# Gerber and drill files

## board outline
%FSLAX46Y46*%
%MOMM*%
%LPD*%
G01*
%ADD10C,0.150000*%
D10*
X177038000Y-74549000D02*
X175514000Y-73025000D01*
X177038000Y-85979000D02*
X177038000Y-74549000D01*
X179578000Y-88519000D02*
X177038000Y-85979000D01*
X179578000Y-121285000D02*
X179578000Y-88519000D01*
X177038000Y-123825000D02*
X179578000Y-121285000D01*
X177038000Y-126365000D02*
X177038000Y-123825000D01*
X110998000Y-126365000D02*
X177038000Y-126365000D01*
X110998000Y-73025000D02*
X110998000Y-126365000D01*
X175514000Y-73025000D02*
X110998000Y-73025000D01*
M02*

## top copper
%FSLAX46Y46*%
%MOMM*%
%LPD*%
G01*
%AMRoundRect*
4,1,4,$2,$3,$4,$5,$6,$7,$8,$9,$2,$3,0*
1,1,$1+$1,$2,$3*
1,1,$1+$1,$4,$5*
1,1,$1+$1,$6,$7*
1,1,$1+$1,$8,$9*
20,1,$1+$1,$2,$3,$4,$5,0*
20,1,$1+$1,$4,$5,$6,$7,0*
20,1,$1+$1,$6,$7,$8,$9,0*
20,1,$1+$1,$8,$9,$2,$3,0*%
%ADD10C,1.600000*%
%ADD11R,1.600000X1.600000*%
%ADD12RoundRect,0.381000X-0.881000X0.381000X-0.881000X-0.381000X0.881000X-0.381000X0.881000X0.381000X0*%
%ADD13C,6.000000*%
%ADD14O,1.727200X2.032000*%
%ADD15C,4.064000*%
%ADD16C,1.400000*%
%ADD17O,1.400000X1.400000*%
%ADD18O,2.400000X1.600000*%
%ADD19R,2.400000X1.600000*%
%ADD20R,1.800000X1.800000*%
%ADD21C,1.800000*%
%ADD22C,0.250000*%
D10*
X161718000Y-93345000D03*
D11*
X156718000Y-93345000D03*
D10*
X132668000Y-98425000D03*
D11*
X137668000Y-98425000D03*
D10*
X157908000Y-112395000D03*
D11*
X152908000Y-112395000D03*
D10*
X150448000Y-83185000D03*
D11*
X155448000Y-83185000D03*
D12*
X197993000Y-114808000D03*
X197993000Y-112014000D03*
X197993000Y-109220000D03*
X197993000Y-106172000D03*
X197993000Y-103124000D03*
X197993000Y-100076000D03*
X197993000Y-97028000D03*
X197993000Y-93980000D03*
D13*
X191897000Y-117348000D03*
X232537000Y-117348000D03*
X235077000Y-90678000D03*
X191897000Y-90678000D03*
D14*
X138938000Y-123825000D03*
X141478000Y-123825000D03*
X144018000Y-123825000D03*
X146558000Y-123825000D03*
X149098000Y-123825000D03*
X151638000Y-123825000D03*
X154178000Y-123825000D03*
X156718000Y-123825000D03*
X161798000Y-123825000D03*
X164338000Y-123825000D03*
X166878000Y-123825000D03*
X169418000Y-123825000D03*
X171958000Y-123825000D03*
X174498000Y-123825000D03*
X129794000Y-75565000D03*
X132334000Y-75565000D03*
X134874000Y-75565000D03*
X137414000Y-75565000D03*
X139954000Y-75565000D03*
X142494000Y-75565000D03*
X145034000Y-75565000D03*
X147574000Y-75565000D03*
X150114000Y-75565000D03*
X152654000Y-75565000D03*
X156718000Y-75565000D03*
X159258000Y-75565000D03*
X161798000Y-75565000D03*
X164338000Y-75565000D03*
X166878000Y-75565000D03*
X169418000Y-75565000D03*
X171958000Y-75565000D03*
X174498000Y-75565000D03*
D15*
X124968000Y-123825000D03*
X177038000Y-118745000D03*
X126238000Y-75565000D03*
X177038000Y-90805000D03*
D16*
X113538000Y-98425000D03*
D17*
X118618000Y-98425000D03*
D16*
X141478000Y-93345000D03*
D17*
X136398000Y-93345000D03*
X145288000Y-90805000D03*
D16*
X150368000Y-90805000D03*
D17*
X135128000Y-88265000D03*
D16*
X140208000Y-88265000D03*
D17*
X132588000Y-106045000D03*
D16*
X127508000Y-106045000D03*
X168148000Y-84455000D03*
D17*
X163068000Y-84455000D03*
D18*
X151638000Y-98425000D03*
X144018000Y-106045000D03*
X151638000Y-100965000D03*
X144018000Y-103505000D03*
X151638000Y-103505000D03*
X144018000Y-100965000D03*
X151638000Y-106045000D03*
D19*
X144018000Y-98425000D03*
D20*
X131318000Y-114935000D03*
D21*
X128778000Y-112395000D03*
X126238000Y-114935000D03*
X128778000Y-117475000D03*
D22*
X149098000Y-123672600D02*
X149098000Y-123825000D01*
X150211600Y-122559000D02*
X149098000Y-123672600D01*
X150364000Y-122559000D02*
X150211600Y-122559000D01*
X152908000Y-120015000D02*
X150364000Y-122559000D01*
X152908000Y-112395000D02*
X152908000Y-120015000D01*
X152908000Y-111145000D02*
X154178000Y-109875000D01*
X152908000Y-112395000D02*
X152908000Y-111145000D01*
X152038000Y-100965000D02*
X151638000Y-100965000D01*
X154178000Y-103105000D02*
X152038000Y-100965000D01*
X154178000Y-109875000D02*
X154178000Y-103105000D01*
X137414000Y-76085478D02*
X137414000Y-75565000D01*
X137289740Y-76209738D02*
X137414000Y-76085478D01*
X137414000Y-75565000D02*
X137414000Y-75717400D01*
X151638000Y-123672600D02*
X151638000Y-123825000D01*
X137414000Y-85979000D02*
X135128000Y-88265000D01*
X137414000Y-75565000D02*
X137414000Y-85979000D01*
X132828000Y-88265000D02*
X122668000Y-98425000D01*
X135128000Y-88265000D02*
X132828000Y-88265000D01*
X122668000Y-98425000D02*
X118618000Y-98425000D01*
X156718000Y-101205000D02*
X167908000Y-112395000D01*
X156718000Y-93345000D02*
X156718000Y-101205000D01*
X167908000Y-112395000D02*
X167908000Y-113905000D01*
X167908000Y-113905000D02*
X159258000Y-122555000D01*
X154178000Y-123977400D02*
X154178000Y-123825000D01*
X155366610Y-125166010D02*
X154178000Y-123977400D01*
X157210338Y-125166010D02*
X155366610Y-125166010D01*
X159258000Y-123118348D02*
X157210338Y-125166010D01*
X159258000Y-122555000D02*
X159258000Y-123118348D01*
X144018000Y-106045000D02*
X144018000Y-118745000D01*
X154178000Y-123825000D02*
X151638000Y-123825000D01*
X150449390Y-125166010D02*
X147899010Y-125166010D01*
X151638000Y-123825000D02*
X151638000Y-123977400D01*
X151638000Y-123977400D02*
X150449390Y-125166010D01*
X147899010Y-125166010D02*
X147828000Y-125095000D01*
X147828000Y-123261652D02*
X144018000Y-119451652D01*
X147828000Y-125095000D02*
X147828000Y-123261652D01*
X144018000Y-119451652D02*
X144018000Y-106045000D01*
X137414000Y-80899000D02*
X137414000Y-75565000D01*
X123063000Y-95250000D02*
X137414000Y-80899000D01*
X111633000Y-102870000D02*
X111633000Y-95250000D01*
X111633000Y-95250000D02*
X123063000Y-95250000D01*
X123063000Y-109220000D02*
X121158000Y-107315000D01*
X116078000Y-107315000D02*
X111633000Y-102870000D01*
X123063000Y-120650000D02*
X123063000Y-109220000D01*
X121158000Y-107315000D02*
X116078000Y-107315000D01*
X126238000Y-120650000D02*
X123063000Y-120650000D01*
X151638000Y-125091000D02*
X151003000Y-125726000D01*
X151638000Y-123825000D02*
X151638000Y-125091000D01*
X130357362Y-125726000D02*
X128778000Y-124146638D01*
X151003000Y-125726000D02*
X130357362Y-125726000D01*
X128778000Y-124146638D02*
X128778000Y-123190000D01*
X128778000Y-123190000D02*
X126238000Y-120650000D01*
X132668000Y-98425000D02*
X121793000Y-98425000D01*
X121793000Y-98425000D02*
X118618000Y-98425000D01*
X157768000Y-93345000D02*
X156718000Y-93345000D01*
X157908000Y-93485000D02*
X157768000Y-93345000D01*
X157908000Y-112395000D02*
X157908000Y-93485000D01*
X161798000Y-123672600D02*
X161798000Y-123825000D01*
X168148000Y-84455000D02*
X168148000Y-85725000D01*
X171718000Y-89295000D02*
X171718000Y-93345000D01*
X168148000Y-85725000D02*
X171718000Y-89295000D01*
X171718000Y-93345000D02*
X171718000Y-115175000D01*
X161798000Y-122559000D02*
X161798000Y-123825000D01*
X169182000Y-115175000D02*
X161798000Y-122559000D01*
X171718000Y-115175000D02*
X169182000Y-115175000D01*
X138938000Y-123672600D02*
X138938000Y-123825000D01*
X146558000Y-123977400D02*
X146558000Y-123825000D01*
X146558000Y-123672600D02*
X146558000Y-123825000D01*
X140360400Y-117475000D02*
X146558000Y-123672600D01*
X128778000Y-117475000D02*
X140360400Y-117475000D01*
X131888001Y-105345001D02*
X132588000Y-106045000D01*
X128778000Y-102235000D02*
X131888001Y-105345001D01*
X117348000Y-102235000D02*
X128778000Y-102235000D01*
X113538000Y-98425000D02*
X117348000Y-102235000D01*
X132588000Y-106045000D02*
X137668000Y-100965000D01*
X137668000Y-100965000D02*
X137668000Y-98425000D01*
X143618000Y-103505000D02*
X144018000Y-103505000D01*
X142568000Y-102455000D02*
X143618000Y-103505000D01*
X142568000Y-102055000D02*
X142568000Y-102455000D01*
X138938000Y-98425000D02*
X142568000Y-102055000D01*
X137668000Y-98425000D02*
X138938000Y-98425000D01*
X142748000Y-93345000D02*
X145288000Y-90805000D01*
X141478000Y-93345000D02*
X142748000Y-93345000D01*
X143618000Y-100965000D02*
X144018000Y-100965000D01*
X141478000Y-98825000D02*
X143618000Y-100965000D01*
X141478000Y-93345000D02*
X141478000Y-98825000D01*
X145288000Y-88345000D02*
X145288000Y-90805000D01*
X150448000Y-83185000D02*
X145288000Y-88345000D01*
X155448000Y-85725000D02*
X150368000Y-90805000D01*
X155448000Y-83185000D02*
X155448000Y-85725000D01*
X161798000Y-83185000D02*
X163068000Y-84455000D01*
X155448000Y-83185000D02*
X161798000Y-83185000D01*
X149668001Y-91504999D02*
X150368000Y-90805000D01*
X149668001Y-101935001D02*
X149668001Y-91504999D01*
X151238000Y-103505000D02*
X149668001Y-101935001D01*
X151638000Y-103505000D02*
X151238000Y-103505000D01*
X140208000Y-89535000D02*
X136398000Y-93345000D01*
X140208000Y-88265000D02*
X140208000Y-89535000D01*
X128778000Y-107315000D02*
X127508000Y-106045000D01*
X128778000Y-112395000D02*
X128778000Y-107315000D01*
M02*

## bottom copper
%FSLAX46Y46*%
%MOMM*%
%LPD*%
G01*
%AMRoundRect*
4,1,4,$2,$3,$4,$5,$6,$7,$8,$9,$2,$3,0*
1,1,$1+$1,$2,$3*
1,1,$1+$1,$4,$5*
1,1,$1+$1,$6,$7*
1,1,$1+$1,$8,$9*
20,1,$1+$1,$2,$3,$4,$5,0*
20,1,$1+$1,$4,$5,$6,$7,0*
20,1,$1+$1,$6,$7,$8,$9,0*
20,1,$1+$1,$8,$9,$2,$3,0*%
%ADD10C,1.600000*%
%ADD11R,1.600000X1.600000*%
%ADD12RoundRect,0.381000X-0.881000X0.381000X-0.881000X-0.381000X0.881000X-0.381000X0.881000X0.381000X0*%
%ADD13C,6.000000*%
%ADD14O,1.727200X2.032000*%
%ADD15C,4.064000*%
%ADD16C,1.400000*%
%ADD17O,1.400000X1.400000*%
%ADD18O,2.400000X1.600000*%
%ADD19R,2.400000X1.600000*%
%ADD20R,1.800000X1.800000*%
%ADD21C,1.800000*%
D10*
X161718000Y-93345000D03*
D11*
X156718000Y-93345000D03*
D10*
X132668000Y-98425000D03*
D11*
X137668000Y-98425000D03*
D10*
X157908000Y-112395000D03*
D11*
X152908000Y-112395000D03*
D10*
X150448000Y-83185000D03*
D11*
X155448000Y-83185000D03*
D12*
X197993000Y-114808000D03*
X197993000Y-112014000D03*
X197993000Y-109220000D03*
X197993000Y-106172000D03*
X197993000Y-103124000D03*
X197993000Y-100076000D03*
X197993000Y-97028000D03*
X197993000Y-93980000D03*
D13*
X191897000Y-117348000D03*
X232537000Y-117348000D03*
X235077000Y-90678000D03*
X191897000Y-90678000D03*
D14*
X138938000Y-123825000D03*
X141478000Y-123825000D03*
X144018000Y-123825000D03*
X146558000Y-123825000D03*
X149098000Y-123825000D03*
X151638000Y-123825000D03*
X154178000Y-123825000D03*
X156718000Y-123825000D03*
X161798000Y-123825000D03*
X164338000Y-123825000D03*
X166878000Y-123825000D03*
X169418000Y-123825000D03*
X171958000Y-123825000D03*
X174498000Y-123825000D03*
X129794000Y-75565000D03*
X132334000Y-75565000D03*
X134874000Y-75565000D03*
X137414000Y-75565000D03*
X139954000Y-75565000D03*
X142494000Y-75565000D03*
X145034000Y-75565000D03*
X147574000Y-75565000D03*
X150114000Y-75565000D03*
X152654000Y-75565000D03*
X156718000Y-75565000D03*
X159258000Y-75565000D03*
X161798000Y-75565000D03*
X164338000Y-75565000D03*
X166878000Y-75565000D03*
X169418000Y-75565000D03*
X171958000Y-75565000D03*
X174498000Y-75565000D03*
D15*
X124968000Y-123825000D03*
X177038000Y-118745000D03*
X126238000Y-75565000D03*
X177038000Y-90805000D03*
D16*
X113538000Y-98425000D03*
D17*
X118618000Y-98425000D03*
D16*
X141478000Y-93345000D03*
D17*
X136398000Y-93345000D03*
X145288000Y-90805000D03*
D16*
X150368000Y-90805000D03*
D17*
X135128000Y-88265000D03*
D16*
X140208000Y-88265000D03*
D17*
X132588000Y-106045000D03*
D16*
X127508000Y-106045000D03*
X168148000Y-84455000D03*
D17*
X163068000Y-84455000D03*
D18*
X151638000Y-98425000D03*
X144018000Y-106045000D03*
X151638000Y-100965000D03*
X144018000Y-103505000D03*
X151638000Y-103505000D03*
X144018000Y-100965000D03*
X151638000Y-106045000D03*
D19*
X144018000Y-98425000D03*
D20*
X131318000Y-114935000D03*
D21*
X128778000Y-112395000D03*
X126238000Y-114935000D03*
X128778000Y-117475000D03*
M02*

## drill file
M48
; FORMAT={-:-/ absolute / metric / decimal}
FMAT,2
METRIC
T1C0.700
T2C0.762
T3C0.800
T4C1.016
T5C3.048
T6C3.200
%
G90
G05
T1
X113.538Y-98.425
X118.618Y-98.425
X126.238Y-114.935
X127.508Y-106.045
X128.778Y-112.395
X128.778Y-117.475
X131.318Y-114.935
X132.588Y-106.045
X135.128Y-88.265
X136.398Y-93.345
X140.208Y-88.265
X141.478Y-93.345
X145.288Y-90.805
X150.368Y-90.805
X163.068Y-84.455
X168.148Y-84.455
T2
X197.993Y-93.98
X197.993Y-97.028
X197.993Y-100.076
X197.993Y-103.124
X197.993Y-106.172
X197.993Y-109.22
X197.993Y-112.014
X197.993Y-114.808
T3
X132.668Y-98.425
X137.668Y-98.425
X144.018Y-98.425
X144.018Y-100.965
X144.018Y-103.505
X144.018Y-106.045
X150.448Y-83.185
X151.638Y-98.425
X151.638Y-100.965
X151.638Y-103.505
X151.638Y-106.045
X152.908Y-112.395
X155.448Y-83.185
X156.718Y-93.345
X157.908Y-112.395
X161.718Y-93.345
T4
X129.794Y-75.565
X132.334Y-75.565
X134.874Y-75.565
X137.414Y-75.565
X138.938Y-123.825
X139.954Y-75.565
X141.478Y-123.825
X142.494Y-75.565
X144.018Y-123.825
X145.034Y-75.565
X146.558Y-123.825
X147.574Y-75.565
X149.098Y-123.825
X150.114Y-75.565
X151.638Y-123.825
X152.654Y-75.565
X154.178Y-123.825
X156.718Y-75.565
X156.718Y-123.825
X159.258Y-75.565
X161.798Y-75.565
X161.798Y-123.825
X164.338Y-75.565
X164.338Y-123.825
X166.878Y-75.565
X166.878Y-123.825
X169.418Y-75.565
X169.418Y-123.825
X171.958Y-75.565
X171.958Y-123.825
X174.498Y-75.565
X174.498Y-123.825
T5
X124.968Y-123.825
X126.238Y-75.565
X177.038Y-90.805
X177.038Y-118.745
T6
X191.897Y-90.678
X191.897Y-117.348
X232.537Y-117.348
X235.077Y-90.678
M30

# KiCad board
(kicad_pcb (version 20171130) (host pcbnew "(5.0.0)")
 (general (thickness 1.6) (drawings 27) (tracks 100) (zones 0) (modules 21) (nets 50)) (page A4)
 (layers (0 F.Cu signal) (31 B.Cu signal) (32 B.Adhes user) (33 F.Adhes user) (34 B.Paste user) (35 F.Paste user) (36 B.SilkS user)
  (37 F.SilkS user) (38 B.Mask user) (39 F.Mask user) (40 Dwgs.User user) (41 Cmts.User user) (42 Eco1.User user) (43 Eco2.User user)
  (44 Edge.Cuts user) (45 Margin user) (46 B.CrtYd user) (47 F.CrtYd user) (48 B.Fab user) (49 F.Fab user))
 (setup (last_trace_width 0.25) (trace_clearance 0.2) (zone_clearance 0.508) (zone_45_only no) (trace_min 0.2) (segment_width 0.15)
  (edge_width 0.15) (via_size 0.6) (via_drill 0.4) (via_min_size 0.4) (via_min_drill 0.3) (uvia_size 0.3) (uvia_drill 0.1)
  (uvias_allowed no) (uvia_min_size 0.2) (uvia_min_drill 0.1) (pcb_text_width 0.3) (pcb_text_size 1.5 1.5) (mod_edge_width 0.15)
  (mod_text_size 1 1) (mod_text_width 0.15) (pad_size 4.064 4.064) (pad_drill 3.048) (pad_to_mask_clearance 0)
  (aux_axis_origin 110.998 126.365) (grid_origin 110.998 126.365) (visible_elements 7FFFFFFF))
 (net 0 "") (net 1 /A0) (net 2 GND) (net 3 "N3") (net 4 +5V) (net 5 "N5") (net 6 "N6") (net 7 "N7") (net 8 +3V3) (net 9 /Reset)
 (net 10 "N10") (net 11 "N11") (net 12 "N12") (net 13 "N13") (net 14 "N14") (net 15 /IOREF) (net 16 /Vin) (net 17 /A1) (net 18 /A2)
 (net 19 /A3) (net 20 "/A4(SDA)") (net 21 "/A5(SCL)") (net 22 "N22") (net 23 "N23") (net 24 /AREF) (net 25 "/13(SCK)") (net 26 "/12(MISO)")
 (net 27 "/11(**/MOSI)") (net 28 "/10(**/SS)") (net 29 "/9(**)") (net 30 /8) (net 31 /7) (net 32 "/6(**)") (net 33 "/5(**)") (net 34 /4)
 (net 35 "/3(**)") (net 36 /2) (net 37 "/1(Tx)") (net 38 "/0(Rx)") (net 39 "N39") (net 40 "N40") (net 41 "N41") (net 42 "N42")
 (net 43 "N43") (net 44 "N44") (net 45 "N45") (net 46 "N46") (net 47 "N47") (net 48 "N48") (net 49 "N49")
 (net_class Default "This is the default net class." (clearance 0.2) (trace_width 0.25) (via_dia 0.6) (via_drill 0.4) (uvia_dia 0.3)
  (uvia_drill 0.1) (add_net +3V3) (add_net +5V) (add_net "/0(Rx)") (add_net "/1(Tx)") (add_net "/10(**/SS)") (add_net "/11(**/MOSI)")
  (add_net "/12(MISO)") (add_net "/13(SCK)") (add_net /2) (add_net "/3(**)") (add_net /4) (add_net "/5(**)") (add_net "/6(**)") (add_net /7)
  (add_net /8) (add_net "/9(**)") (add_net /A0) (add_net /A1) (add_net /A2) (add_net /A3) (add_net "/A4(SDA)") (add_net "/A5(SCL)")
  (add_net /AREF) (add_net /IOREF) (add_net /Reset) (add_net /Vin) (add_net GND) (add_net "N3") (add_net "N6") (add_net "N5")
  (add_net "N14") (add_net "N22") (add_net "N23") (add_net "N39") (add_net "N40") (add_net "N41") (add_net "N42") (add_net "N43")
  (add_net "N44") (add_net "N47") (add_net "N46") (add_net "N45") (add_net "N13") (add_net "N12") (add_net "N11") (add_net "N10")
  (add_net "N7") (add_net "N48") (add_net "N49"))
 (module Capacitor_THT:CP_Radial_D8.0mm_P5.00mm (layer F.Cu) (at 156.718 93.345)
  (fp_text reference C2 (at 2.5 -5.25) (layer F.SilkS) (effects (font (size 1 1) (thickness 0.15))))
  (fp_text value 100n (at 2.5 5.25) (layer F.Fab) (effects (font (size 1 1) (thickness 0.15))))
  (pad 2 thru_hole circle (at 5 0) (size 1.6 1.6) (drill 0.8) (layers *.Cu *.Mask) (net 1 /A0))
  (pad 1 thru_hole rect (at 0 0) (size 1.6 1.6) (drill 0.8) (layers *.Cu *.Mask) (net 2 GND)))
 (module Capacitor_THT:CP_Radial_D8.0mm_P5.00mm (layer F.Cu) (at 137.668 98.425 180)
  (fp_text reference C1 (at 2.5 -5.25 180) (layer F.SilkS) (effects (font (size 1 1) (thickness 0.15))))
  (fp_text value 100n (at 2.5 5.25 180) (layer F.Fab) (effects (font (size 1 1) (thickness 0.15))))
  (pad 2 thru_hole circle (at 5 0 180) (size 1.6 1.6) (drill 0.8) (layers *.Cu *.Mask) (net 2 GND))
  (pad 1 thru_hole rect (at 0 0 180) (size 1.6 1.6) (drill 0.8) (layers *.Cu *.Mask) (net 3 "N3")))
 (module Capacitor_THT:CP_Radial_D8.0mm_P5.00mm (layer F.Cu) (at 152.908 112.395)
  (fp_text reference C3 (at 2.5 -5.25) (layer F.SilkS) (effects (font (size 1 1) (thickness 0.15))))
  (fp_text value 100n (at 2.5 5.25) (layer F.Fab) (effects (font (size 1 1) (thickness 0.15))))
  (pad 2 thru_hole circle (at 5 0) (size 1.6 1.6) (drill 0.8) (layers *.Cu *.Mask) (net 2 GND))
  (pad 1 thru_hole rect (at 0 0) (size 1.6 1.6) (drill 0.8) (layers *.Cu *.Mask) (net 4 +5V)))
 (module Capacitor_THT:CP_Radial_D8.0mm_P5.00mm (layer F.Cu) (at 155.448 83.185 180)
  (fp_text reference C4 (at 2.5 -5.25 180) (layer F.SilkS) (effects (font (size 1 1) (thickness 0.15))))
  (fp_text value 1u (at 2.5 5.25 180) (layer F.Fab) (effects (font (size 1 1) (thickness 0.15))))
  (pad 2 thru_hole circle (at 5 0 180) (size 1.6 1.6) (drill 0.8) (layers *.Cu *.Mask) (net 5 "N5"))
  (pad 1 thru_hole rect (at 0 0 180) (size 1.6 1.6) (drill 0.8) (layers *.Cu *.Mask) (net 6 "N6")))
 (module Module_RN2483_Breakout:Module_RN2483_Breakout (layer F.Cu) (at 197.993 93.98 270)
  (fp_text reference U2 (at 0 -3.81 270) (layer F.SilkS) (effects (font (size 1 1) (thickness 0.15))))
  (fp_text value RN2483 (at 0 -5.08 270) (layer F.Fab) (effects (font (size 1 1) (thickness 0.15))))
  (pad 8 thru_hole roundrect (at 20.828 0 270) (size 1.524 2.524) (drill 0.762) (layers *.Cu *.Mask) (roundrect_rratio 0.25) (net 2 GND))
  (pad 7 thru_hole roundrect (at 18.034 0 270) (size 1.524 2.524) (drill 0.762) (layers *.Cu *.Mask) (roundrect_rratio 0.25) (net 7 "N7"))
  (pad 6 thru_hole roundrect (at 15.24 0 270) (size 1.524 2.524) (drill 0.762) (layers *.Cu *.Mask) (roundrect_rratio 0.25) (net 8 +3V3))
  (pad 5 thru_hole roundrect (at 12.192 0 270) (size 1.524 2.524) (drill 0.762) (layers *.Cu *.Mask) (roundrect_rratio 0.25) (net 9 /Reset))
  (pad 4 thru_hole roundrect (at 9.144 0 270) (size 1.524 2.524) (drill 0.762) (layers *.Cu *.Mask) (roundrect_rratio 0.25) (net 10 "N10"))
  (pad 3 thru_hole roundrect (at 6.096 0 270) (size 1.524 2.524) (drill 0.762) (layers *.Cu *.Mask) (roundrect_rratio 0.25) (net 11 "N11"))
  (pad 2 thru_hole roundrect (at 3.048 0 270) (size 1.524 2.524) (drill 0.762) (layers *.Cu *.Mask) (roundrect_rratio 0.25) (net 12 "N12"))
  (pad 1 thru_hole roundrect (at 0 0 270) (size 1.524 2.524) (drill 0.762) (layers *.Cu *.Mask) (roundrect_rratio 0.25) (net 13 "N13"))
  (pad "" thru_hole circle (at 23.368 6.096 270) (size 6 6) (drill 3.2) (layers *.Cu *.Mask))
  (pad "" thru_hole circle (at 23.368 -34.544 270) (size 6 6) (drill 3.2) (layers *.Cu *.Mask))
  (pad "" thru_hole circle (at -3.302 -37.084 270) (size 6 6) (drill 3.2) (layers *.Cu *.Mask))
  (pad "" thru_hole circle (at -3.302 6.096 270) (size 6 6) (drill 3.2) (layers *.Cu *.Mask)))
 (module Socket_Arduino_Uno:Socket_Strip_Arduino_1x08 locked (layer F.Cu) (at 138.938 123.825)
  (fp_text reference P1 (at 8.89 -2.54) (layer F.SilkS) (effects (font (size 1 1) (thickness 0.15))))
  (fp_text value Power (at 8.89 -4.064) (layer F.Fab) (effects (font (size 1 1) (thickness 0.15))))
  (pad 1 thru_hole oval (at 0 0) (size 1.7272 2.032) (drill 1.016) (layers *.Cu *.Mask F.SilkS) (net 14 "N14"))
  (pad 2 thru_hole oval (at 2.54 0) (size 1.7272 2.032) (drill 1.016) (layers *.Cu *.Mask F.SilkS) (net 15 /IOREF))
  (pad 3 thru_hole oval (at 5.08 0) (size 1.7272 2.032) (drill 1.016) (layers *.Cu *.Mask F.SilkS) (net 9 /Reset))
  (pad 4 thru_hole oval (at 7.62 0) (size 1.7272 2.032) (drill 1.016) (layers *.Cu *.Mask F.SilkS) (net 8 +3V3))
  (pad 5 thru_hole oval (at 10.16 0) (size 1.7272 2.032) (drill 1.016) (layers *.Cu *.Mask F.SilkS) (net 4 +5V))
  (pad 6 thru_hole oval (at 12.7 0) (size 1.7272 2.032) (drill 1.016) (layers *.Cu *.Mask F.SilkS) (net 2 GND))
  (pad 7 thru_hole oval (at 15.24 0) (size 1.7272 2.032) (drill 1.016) (layers *.Cu *.Mask F.SilkS) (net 2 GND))
  (pad 8 thru_hole oval (at 17.78 0) (size 1.7272 2.032) (drill 1.016) (layers *.Cu *.Mask F.SilkS) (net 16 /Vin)))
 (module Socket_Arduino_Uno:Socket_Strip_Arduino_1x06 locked (layer F.Cu) (at 161.798 123.825)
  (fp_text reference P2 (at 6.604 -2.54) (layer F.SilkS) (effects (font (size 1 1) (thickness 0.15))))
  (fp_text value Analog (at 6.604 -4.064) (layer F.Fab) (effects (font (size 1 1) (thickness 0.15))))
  (pad 1 thru_hole oval (at 0 0) (size 1.7272 2.032) (drill 1.016) (layers *.Cu *.Mask F.SilkS) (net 1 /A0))
  (pad 2 thru_hole oval (at 2.54 0) (size 1.7272 2.032) (drill 1.016) (layers *.Cu *.Mask F.SilkS) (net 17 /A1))
  (pad 3 thru_hole oval (at 5.08 0) (size 1.7272 2.032) (drill 1.016) (layers *.Cu *.Mask F.SilkS) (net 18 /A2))
  (pad 4 thru_hole oval (at 7.62 0) (size 1.7272 2.032) (drill 1.016) (layers *.Cu *.Mask F.SilkS) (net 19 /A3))
  (pad 5 thru_hole oval (at 10.16 0) (size 1.7272 2.032) (drill 1.016) (layers *.Cu *.Mask F.SilkS) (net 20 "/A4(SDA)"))
  (pad 6 thru_hole oval (at 12.7 0) (size 1.7272 2.032) (drill 1.016) (layers *.Cu *.Mask F.SilkS) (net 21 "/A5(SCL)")))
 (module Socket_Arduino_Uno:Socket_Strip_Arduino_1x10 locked (layer F.Cu) (at 129.794 75.565)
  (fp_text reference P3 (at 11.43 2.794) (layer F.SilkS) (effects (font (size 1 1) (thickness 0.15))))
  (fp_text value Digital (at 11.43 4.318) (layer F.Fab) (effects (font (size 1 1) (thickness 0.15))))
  (pad 1 thru_hole oval (at 0 0) (size 1.7272 2.032) (drill 1.016) (layers *.Cu *.Mask F.SilkS) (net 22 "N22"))
  (pad 2 thru_hole oval (at 2.54 0) (size 1.7272 2.032) (drill 1.016) (layers *.Cu *.Mask F.SilkS) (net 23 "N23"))
  (pad 3 thru_hole oval (at 5.08 0) (size 1.7272 2.032) (drill 1.016) (layers *.Cu *.Mask F.SilkS) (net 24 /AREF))
  (pad 4 thru_hole oval (at 7.62 0) (size 1.7272 2.032) (drill 1.016) (layers *.Cu *.Mask F.SilkS) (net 2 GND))
  (pad 5 thru_hole oval (at 10.16 0) (size 1.7272 2.032) (drill 1.016) (layers *.Cu *.Mask F.SilkS) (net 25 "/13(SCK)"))
  (pad 6 thru_hole oval (at 12.7 0) (size 1.7272 2.032) (drill 1.016) (layers *.Cu *.Mask F.SilkS) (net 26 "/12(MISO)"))
  (pad 7 thru_hole oval (at 15.24 0) (size 1.7272 2.032) (drill 1.016) (layers *.Cu *.Mask F.SilkS) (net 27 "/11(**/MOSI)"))
  (pad 8 thru_hole oval (at 17.78 0) (size 1.7272 2.032) (drill 1.016) (layers *.Cu *.Mask F.SilkS) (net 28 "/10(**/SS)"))
  (pad 9 thru_hole oval (at 20.32 0) (size 1.7272 2.032) (drill 1.016) (layers *.Cu *.Mask F.SilkS) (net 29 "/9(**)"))
  (pad 10 thru_hole oval (at 22.86 0) (size 1.7272 2.032) (drill 1.016) (layers *.Cu *.Mask F.SilkS) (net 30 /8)))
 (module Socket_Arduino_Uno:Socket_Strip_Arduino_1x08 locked (layer F.Cu) (at 156.718 75.565)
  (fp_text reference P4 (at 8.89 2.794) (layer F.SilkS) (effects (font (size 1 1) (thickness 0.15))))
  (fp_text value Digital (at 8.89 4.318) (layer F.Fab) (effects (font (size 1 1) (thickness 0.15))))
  (pad 1 thru_hole oval (at 0 0) (size 1.7272 2.032) (drill 1.016) (layers *.Cu *.Mask F.SilkS) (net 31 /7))
  (pad 2 thru_hole oval (at 2.54 0) (size 1.7272 2.032) (drill 1.016) (layers *.Cu *.Mask F.SilkS) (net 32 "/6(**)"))
  (pad 3 thru_hole oval (at 5.08 0) (size 1.7272 2.032) (drill 1.016) (layers *.Cu *.Mask F.SilkS) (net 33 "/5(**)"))
  (pad 4 thru_hole oval (at 7.62 0) (size 1.7272 2.032) (drill 1.016) (layers *.Cu *.Mask F.SilkS) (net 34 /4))
  (pad 5 thru_hole oval (at 10.16 0) (size 1.7272 2.032) (drill 1.016) (layers *.Cu *.Mask F.SilkS) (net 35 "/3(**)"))
  (pad 6 thru_hole oval (at 12.7 0) (size 1.7272 2.032) (drill 1.016) (layers *.Cu *.Mask F.SilkS) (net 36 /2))
  (pad 7 thru_hole oval (at 15.24 0) (size 1.7272 2.032) (drill 1.016) (layers *.Cu *.Mask F.SilkS) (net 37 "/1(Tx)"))
  (pad 8 thru_hole oval (at 17.78 0) (size 1.7272 2.032) (drill 1.016) (layers *.Cu *.Mask F.SilkS) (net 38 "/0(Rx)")))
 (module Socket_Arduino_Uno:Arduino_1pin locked (layer F.Cu) (at 124.968 123.825)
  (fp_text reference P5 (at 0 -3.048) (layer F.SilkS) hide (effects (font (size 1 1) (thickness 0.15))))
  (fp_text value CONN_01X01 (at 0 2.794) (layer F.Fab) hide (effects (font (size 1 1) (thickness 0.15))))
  (pad 1 thru_hole circle (at 0 0) (size 4.064 4.064) (drill 3.048) (layers *.Cu *.Mask F.SilkS) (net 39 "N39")))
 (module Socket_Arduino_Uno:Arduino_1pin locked (layer F.Cu) (at 177.038 118.745)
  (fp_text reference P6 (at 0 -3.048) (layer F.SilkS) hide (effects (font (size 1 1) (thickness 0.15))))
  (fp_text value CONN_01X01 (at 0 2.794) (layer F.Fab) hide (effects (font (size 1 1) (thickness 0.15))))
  (pad 1 thru_hole circle (at 0 0) (size 4.064 4.064) (drill 3.048) (layers *.Cu *.Mask F.SilkS) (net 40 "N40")))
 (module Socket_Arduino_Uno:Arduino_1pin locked (layer F.Cu) (at 126.238 75.565)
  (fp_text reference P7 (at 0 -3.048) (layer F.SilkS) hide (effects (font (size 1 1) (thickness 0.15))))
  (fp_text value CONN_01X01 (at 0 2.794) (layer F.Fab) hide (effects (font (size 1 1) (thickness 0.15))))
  (pad 1 thru_hole circle (at 0 0) (size 4.064 4.064) (drill 3.048) (layers *.Cu *.Mask F.SilkS) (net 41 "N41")))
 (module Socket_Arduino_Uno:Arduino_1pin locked (layer F.Cu) (at 177.038 90.805)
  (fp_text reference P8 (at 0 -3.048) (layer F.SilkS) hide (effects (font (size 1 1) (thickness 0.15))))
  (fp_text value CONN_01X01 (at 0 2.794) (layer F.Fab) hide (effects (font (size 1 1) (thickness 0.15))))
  (pad 1 thru_hole circle (at 0 0) (size 4.064 4.064) (drill 3.048) (layers *.Cu *.Mask F.SilkS) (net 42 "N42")))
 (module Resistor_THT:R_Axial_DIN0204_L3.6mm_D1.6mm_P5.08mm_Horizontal (layer F.Cu) (at 113.538 98.425)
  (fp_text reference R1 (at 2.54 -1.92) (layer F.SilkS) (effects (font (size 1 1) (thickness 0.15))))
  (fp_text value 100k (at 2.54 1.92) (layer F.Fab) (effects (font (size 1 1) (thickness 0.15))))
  (pad 1 thru_hole circle (at 0 0) (size 1.4 1.4) (drill 0.7) (layers *.Cu *.Mask) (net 3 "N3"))
  (pad 2 thru_hole oval (at 5.08 0) (size 1.4 1.4) (drill 0.7) (layers *.Cu *.Mask) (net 2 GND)))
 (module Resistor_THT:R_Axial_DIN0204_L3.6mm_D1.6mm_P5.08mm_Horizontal (layer F.Cu) (at 141.478 93.345 180)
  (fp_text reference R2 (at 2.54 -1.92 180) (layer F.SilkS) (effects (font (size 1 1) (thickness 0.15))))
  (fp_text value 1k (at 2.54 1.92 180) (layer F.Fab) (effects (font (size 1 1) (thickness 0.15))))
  (pad 1 thru_hole circle (at 0 0 180) (size 1.4 1.4) (drill 0.7) (layers *.Cu *.Mask) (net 5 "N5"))
  (pad 2 thru_hole oval (at 5.08 0 180) (size 1.4 1.4) (drill 0.7) (layers *.Cu *.Mask) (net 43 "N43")))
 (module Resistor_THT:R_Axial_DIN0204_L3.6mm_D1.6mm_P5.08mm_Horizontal (layer F.Cu) (at 150.368 90.805 180)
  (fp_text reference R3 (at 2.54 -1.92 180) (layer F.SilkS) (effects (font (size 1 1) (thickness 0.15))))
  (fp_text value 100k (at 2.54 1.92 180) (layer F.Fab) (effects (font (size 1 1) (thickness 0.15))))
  (pad 2 thru_hole oval (at 5.08 0 180) (size 1.4 1.4) (drill 0.7) (layers *.Cu *.Mask) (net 5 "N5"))
  (pad 1 thru_hole circle (at 0 0 180) (size 1.4 1.4) (drill 0.7) (layers *.Cu *.Mask) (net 6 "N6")))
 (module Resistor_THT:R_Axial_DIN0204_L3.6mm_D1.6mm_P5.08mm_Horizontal (layer F.Cu) (at 140.208 88.265 180)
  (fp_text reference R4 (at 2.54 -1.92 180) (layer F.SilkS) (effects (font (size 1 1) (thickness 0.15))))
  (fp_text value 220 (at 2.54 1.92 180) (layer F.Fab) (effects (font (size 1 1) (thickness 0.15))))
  (pad 2 thru_hole oval (at 5.08 0 180) (size 1.4 1.4) (drill 0.7) (layers *.Cu *.Mask) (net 2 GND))
  (pad 1 thru_hole circle (at 0 0 180) (size 1.4 1.4) (drill 0.7) (layers *.Cu *.Mask) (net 43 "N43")))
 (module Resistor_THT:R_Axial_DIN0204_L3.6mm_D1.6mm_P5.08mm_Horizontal (layer F.Cu) (at 127.508 106.045)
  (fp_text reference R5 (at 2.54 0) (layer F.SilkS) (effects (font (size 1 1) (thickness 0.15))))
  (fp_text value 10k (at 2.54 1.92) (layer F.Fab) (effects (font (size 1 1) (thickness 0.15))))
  (pad 2 thru_hole oval (at 5.08 0) (size 1.4 1.4) (drill 0.7) (layers *.Cu *.Mask) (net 3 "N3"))
  (pad 1 thru_hole circle (at 0 0) (size 1.4 1.4) (drill 0.7) (layers *.Cu *.Mask) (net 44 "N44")))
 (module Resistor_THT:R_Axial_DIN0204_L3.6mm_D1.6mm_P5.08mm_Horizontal (layer F.Cu) (at 168.148 84.455 180)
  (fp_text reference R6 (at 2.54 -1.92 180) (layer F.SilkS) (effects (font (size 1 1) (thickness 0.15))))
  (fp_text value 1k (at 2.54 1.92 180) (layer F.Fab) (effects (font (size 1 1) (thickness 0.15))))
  (pad 1 thru_hole circle (at 0 0 180) (size 1.4 1.4) (drill 0.7) (layers *.Cu *.Mask) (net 1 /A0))
  (pad 2 thru_hole oval (at 5.08 0 180) (size 1.4 1.4) (drill 0.7) (layers *.Cu *.Mask) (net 6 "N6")))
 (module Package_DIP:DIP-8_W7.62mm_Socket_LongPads (layer F.Cu) (at 144.018 98.425)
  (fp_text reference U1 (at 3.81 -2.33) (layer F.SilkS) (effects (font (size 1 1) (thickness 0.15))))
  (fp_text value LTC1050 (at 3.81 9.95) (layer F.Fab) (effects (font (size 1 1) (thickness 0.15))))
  (pad 8 thru_hole oval (at 7.62 0) (size 2.4 1.6) (drill 0.8) (layers *.Cu *.Mask) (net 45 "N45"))
  (pad 4 thru_hole oval (at 0 7.62) (size 2.4 1.6) (drill 0.8) (layers *.Cu *.Mask) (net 2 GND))
  (pad 7 thru_hole oval (at 7.62 2.54) (size 2.4 1.6) (drill 0.8) (layers *.Cu *.Mask) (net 4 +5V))
  (pad 3 thru_hole oval (at 0 5.08) (size 2.4 1.6) (drill 0.8) (layers *.Cu *.Mask) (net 3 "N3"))
  (pad 6 thru_hole oval (at 7.62 5.08) (size 2.4 1.6) (drill 0.8) (layers *.Cu *.Mask) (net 6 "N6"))
  (pad 2 thru_hole oval (at 0 2.54) (size 2.4 1.6) (drill 0.8) (layers *.Cu *.Mask) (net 5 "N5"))
  (pad 5 thru_hole oval (at 7.62 7.62) (size 2.4 1.6) (drill 0.8) (layers *.Cu *.Mask) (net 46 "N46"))
  (pad 1 thru_hole rect (at 0 0) (size 2.4 1.6) (drill 0.8) (layers *.Cu *.Mask) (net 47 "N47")))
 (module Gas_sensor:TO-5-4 (layer F.Cu) (at 131.318 114.935 180)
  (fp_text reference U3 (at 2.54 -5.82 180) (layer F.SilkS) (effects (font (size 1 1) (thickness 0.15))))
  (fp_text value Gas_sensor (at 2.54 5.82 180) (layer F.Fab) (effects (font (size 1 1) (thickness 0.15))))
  (pad 1 thru_hole rect (at 0 0 180) (size 1.8 1.8) (drill 0.7) (layers *.Cu *.Mask) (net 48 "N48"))
  (pad 2 thru_hole circle (at 2.54 2.54 180) (size 1.8 1.8) (drill 0.7) (layers *.Cu *.Mask) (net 44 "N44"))
  (pad 3 thru_hole circle (at 5.08 0 180) (size 1.8 1.8) (drill 0.7) (layers *.Cu *.Mask) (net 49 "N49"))
  (pad 4 thru_hole circle (at 2.54 -2.54 180) (size 1.8 1.8) (drill 0.7) (layers *.Cu *.Mask) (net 8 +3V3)))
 (gr_line (start 177.038 74.549) (end 175.514 73.025) (angle 90) (layer Edge.Cuts) (width 0.15))
 (gr_line (start 177.038 85.979) (end 177.038 74.549) (angle 90) (layer Edge.Cuts) (width 0.15))
 (gr_line (start 179.578 88.519) (end 177.038 85.979) (angle 90) (layer Edge.Cuts) (width 0.15))
 (gr_line (start 179.578 121.285) (end 179.578 88.519) (angle 90) (layer Edge.Cuts) (width 0.15))
 (gr_line (start 177.038 123.825) (end 179.578 121.285) (angle 90) (layer Edge.Cuts) (width 0.15))
 (gr_line (start 177.038 126.365) (end 177.038 123.825) (angle 90) (layer Edge.Cuts) (width 0.15))
 (gr_line (start 110.998 126.365) (end 177.038 126.365) (angle 90) (layer Edge.Cuts) (width 0.15))
 (gr_line (start 110.998 73.025) (end 110.998 126.365) (angle 90) (layer Edge.Cuts) (width 0.15))
 (gr_line (start 175.514 73.025) (end 110.998 73.025) (angle 90) (layer Edge.Cuts) (width 0.15))
 (segment (start 149.098 123.6726) (end 149.098 123.825) (width 0.25) (layer F.Cu) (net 4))
 (segment (start 150.2116 122.559) (end 149.098 123.6726) (width 0.25) (layer F.Cu) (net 4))
 (segment (start 150.364 122.559) (end 150.2116 122.559) (width 0.25) (layer F.Cu) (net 4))
 (segment (start 152.908 120.015) (end 150.364 122.559) (width 0.25) (layer F.Cu) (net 4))
 (segment (start 152.908 112.395) (end 152.908 120.015) (width 0.25) (layer F.Cu) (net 4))
 (segment (start 152.908 111.145) (end 154.178 109.875) (width 0.25) (layer F.Cu) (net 4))
 (segment (start 152.908 112.395) (end 152.908 111.145) (width 0.25) (layer F.Cu) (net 4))
 (segment (start 152.038 100.965) (end 151.638 100.965) (width 0.25) (layer F.Cu) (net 4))
 (segment (start 154.178 103.105) (end 152.038 100.965) (width 0.25) (layer F.Cu) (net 4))
 (segment (start 154.178 109.875) (end 154.178 103.105) (width 0.25) (layer F.Cu) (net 4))
 (segment (start 137.414 76.085478) (end 137.414 75.565) (width 0.25) (layer F.Cu) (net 2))
 (segment (start 137.28974 76.209738) (end 137.414 76.085478) (width 0.25) (layer F.Cu) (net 2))
 (segment (start 137.414 75.565) (end 137.414 75.7174) (width 0.25) (layer F.Cu) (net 2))
 (segment (start 151.638 123.6726) (end 151.638 123.825) (width 0.25) (layer F.Cu) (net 2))
 (segment (start 137.414 85.979) (end 135.128 88.265) (width 0.25) (layer F.Cu) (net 2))
 (segment (start 137.414 75.565) (end 137.414 85.979) (width 0.25) (layer F.Cu) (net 2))
 (segment (start 132.828 88.265) (end 122.668 98.425) (width 0.25) (layer F.Cu) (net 2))
 (segment (start 135.128 88.265) (end 132.828 88.265) (width 0.25) (layer F.Cu) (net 2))
 (segment (start 122.668 98.425) (end 118.618 98.425) (width 0.25) (layer F.Cu) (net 2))
 (segment (start 156.718 101.205) (end 167.908 112.395) (width 0.25) (layer F.Cu) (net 2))
 (segment (start 156.718 93.345) (end 156.718 101.205) (width 0.25) (layer F.Cu) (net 2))
 (segment (start 167.908 112.395) (end 167.908 113.905) (width 0.25) (layer F.Cu) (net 2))
 (segment (start 167.908 113.905) (end 159.258 122.555) (width 0.25) (layer F.Cu) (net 2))
 (segment (start 154.178 123.9774) (end 154.178 123.825) (width 0.25) (layer F.Cu) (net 2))
 (segment (start 155.36661 125.16601) (end 154.178 123.9774) (width 0.25) (layer F.Cu) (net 2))
 (segment (start 157.210338 125.16601) (end 155.36661 125.16601) (width 0.25) (layer F.Cu) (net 2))
 (segment (start 159.258 123.118348) (end 157.210338 125.16601) (width 0.25) (layer F.Cu) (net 2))
 (segment (start 159.258 122.555) (end 159.258 123.118348) (width 0.25) (layer F.Cu) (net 2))
 (segment (start 144.018 106.045) (end 144.018 118.745) (width 0.25) (layer F.Cu) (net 2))
 (segment (start 154.178 123.825) (end 151.638 123.825) (width 0.25) (layer F.Cu) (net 2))
 (segment (start 150.44939 125.16601) (end 147.89901 125.16601) (width 0.25) (layer F.Cu) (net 2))
 (segment (start 151.638 123.825) (end 151.638 123.9774) (width 0.25) (layer F.Cu) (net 2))
 (segment (start 151.638 123.9774) (end 150.44939 125.16601) (width 0.25) (layer F.Cu) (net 2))
 (segment (start 147.89901 125.16601) (end 147.828 125.095) (width 0.25) (layer F.Cu) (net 2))
 (segment (start 147.828 123.261652) (end 144.018 119.451652) (width 0.25) (layer F.Cu) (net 2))
 (segment (start 147.828 125.095) (end 147.828 123.261652) (width 0.25) (layer F.Cu) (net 2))
 (segment (start 144.018 119.451652) (end 144.018 106.045) (width 0.25) (layer F.Cu) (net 2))
 (segment (start 137.414 80.899) (end 137.414 75.565) (width 0.25) (layer F.Cu) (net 2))
 (segment (start 123.063 95.25) (end 137.414 80.899) (width 0.25) (layer F.Cu) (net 2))
 (segment (start 111.633 102.87) (end 111.633 95.25) (width 0.25) (layer F.Cu) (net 2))
 (segment (start 111.633 95.25) (end 123.063 95.25) (width 0.25) (layer F.Cu) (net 2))
 (segment (start 123.063 109.22) (end 121.158 107.315) (width 0.25) (layer F.Cu) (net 2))
 (segment (start 116.078 107.315) (end 111.633 102.87) (width 0.25) (layer F.Cu) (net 2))
 (segment (start 123.063 120.65) (end 123.063 109.22) (width 0.25) (layer F.Cu) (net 2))
 (segment (start 121.158 107.315) (end 116.078 107.315) (width 0.25) (layer F.Cu) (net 2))
 (segment (start 126.238 120.65) (end 123.063 120.65) (width 0.25) (layer F.Cu) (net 2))
 (segment (start 151.638 125.091) (end 151.003 125.726) (width 0.25) (layer F.Cu) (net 2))
 (segment (start 151.638 123.825) (end 151.638 125.091) (width 0.25) (layer F.Cu) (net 2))
 (segment (start 130.357362 125.726) (end 128.778 124.146638) (width 0.25) (layer F.Cu) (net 2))
 (segment (start 151.003 125.726) (end 130.357362 125.726) (width 0.25) (layer F.Cu) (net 2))
 (segment (start 128.778 124.146638) (end 128.778 123.19) (width 0.25) (layer F.Cu) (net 2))
 (segment (start 128.778 123.19) (end 126.238 120.65) (width 0.25) (layer F.Cu) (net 2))
 (segment (start 132.668 98.425) (end 121.793 98.425) (width 0.25) (layer F.Cu) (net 2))
 (segment (start 121.793 98.425) (end 118.618 98.425) (width 0.25) (layer F.Cu) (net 2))
 (segment (start 157.768 93.345) (end 156.718 93.345) (width 0.25) (layer F.Cu) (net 2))
 (segment (start 157.908 93.485) (end 157.768 93.345) (width 0.25) (layer F.Cu) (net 2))
 (segment (start 157.908 112.395) (end 157.908 93.485) (width 0.25) (layer F.Cu) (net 2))
 (segment (start 161.798 123.6726) (end 161.798 123.825) (width 0.25) (layer F.Cu) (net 1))
 (segment (start 168.148 84.455) (end 168.148 85.725) (width 0.25) (layer F.Cu) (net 1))
 (segment (start 171.718 89.295) (end 171.718 93.345) (width 0.25) (layer F.Cu) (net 1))
 (segment (start 168.148 85.725) (end 171.718 89.295) (width 0.25) (layer F.Cu) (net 1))
 (segment (start 171.718 93.345) (end 171.718 115.175) (width 0.25) (layer F.Cu) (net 1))
 (segment (start 161.798 122.559) (end 161.798 123.825) (width 0.25) (layer F.Cu) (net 1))
 (segment (start 169.182 115.175) (end 161.798 122.559) (width 0.25) (layer F.Cu) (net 1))
 (segment (start 171.718 115.175) (end 169.182 115.175) (width 0.25) (layer F.Cu) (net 1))
 (segment (start 138.938 123.6726) (end 138.938 123.825) (width 0.25) (layer F.Cu) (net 14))
 (segment (start 146.558 123.9774) (end 146.558 123.825) (width 0.25) (layer F.Cu) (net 8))
 (segment (start 146.558 123.6726) (end 146.558 123.825) (width 0.25) (layer F.Cu) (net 8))
 (segment (start 140.3604 117.475) (end 146.558 123.6726) (width 0.25) (layer F.Cu) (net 8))
 (segment (start 128.778 117.475) (end 140.3604 117.475) (width 0.25) (layer F.Cu) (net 8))
 (segment (start 131.888001 105.345001) (end 132.588 106.045) (width 0.25) (layer F.Cu) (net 3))
 (segment (start 128.778 102.235) (end 131.888001 105.345001) (width 0.25) (layer F.Cu) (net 3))
 (segment (start 117.348 102.235) (end 128.778 102.235) (width 0.25) (layer F.Cu) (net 3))
 (segment (start 113.538 98.425) (end 117.348 102.235) (width 0.25) (layer F.Cu) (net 3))
 (segment (start 132.588 106.045) (end 137.668 100.965) (width 0.25) (layer F.Cu) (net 3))
 (segment (start 137.668 100.965) (end 137.668 98.425) (width 0.25) (layer F.Cu) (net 3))
 (segment (start 143.618 103.505) (end 144.018 103.505) (width 0.25) (layer F.Cu) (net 3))
 (segment (start 142.568 102.455) (end 143.618 103.505) (width 0.25) (layer F.Cu) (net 3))
 (segment (start 142.568 102.055) (end 142.568 102.455) (width 0.25) (layer F.Cu) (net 3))
 (segment (start 138.938 98.425) (end 142.568 102.055) (width 0.25) (layer F.Cu) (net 3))
 (segment (start 137.668 98.425) (end 138.938 98.425) (width 0.25) (layer F.Cu) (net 3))
 (segment (start 142.748 93.345) (end 145.288 90.805) (width 0.25) (layer F.Cu) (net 5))
 (segment (start 141.478 93.345) (end 142.748 93.345) (width 0.25) (layer F.Cu) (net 5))
 (segment (start 143.618 100.965) (end 144.018 100.965) (width 0.25) (layer F.Cu) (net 5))
 (segment (start 141.478 98.825) (end 143.618 100.965) (width 0.25) (layer F.Cu) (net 5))
 (segment (start 141.478 93.345) (end 141.478 98.825) (width 0.25) (layer F.Cu) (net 5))
 (segment (start 145.288 88.345) (end 145.288 90.805) (width 0.25) (layer F.Cu) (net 5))
 (segment (start 150.448 83.185) (end 145.288 88.345) (width 0.25) (layer F.Cu) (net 5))
 (segment (start 155.448 85.725) (end 150.368 90.805) (width 0.25) (layer F.Cu) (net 6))
 (segment (start 155.448 83.185) (end 155.448 85.725) (width 0.25) (layer F.Cu) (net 6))
 (segment (start 161.798 83.185) (end 163.068 84.455) (width 0.25) (layer F.Cu) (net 6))
 (segment (start 155.448 83.185) (end 161.798 83.185) (width 0.25) (layer F.Cu) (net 6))
 (segment (start 149.668001 91.504999) (end 150.368 90.805) (width 0.25) (layer F.Cu) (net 6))
 (segment (start 149.668001 101.935001) (end 149.668001 91.504999) (width 0.25) (layer F.Cu) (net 6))
 (segment (start 151.238 103.505) (end 149.668001 101.935001) (width 0.25) (layer F.Cu) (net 6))
 (segment (start 151.638 103.505) (end 151.238 103.505) (width 0.25) (layer F.Cu) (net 6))
 (segment (start 140.208 89.535) (end 136.398 93.345) (width 0.25) (layer F.Cu) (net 43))
 (segment (start 140.208 88.265) (end 140.208 89.535) (width 0.25) (layer F.Cu) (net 43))
 (segment (start 128.778 107.315) (end 127.508 106.045) (width 0.25) (layer F.Cu) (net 44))
 (segment (start 128.778 112.395) (end 128.778 107.315) (width 0.25) (layer F.Cu) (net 44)))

